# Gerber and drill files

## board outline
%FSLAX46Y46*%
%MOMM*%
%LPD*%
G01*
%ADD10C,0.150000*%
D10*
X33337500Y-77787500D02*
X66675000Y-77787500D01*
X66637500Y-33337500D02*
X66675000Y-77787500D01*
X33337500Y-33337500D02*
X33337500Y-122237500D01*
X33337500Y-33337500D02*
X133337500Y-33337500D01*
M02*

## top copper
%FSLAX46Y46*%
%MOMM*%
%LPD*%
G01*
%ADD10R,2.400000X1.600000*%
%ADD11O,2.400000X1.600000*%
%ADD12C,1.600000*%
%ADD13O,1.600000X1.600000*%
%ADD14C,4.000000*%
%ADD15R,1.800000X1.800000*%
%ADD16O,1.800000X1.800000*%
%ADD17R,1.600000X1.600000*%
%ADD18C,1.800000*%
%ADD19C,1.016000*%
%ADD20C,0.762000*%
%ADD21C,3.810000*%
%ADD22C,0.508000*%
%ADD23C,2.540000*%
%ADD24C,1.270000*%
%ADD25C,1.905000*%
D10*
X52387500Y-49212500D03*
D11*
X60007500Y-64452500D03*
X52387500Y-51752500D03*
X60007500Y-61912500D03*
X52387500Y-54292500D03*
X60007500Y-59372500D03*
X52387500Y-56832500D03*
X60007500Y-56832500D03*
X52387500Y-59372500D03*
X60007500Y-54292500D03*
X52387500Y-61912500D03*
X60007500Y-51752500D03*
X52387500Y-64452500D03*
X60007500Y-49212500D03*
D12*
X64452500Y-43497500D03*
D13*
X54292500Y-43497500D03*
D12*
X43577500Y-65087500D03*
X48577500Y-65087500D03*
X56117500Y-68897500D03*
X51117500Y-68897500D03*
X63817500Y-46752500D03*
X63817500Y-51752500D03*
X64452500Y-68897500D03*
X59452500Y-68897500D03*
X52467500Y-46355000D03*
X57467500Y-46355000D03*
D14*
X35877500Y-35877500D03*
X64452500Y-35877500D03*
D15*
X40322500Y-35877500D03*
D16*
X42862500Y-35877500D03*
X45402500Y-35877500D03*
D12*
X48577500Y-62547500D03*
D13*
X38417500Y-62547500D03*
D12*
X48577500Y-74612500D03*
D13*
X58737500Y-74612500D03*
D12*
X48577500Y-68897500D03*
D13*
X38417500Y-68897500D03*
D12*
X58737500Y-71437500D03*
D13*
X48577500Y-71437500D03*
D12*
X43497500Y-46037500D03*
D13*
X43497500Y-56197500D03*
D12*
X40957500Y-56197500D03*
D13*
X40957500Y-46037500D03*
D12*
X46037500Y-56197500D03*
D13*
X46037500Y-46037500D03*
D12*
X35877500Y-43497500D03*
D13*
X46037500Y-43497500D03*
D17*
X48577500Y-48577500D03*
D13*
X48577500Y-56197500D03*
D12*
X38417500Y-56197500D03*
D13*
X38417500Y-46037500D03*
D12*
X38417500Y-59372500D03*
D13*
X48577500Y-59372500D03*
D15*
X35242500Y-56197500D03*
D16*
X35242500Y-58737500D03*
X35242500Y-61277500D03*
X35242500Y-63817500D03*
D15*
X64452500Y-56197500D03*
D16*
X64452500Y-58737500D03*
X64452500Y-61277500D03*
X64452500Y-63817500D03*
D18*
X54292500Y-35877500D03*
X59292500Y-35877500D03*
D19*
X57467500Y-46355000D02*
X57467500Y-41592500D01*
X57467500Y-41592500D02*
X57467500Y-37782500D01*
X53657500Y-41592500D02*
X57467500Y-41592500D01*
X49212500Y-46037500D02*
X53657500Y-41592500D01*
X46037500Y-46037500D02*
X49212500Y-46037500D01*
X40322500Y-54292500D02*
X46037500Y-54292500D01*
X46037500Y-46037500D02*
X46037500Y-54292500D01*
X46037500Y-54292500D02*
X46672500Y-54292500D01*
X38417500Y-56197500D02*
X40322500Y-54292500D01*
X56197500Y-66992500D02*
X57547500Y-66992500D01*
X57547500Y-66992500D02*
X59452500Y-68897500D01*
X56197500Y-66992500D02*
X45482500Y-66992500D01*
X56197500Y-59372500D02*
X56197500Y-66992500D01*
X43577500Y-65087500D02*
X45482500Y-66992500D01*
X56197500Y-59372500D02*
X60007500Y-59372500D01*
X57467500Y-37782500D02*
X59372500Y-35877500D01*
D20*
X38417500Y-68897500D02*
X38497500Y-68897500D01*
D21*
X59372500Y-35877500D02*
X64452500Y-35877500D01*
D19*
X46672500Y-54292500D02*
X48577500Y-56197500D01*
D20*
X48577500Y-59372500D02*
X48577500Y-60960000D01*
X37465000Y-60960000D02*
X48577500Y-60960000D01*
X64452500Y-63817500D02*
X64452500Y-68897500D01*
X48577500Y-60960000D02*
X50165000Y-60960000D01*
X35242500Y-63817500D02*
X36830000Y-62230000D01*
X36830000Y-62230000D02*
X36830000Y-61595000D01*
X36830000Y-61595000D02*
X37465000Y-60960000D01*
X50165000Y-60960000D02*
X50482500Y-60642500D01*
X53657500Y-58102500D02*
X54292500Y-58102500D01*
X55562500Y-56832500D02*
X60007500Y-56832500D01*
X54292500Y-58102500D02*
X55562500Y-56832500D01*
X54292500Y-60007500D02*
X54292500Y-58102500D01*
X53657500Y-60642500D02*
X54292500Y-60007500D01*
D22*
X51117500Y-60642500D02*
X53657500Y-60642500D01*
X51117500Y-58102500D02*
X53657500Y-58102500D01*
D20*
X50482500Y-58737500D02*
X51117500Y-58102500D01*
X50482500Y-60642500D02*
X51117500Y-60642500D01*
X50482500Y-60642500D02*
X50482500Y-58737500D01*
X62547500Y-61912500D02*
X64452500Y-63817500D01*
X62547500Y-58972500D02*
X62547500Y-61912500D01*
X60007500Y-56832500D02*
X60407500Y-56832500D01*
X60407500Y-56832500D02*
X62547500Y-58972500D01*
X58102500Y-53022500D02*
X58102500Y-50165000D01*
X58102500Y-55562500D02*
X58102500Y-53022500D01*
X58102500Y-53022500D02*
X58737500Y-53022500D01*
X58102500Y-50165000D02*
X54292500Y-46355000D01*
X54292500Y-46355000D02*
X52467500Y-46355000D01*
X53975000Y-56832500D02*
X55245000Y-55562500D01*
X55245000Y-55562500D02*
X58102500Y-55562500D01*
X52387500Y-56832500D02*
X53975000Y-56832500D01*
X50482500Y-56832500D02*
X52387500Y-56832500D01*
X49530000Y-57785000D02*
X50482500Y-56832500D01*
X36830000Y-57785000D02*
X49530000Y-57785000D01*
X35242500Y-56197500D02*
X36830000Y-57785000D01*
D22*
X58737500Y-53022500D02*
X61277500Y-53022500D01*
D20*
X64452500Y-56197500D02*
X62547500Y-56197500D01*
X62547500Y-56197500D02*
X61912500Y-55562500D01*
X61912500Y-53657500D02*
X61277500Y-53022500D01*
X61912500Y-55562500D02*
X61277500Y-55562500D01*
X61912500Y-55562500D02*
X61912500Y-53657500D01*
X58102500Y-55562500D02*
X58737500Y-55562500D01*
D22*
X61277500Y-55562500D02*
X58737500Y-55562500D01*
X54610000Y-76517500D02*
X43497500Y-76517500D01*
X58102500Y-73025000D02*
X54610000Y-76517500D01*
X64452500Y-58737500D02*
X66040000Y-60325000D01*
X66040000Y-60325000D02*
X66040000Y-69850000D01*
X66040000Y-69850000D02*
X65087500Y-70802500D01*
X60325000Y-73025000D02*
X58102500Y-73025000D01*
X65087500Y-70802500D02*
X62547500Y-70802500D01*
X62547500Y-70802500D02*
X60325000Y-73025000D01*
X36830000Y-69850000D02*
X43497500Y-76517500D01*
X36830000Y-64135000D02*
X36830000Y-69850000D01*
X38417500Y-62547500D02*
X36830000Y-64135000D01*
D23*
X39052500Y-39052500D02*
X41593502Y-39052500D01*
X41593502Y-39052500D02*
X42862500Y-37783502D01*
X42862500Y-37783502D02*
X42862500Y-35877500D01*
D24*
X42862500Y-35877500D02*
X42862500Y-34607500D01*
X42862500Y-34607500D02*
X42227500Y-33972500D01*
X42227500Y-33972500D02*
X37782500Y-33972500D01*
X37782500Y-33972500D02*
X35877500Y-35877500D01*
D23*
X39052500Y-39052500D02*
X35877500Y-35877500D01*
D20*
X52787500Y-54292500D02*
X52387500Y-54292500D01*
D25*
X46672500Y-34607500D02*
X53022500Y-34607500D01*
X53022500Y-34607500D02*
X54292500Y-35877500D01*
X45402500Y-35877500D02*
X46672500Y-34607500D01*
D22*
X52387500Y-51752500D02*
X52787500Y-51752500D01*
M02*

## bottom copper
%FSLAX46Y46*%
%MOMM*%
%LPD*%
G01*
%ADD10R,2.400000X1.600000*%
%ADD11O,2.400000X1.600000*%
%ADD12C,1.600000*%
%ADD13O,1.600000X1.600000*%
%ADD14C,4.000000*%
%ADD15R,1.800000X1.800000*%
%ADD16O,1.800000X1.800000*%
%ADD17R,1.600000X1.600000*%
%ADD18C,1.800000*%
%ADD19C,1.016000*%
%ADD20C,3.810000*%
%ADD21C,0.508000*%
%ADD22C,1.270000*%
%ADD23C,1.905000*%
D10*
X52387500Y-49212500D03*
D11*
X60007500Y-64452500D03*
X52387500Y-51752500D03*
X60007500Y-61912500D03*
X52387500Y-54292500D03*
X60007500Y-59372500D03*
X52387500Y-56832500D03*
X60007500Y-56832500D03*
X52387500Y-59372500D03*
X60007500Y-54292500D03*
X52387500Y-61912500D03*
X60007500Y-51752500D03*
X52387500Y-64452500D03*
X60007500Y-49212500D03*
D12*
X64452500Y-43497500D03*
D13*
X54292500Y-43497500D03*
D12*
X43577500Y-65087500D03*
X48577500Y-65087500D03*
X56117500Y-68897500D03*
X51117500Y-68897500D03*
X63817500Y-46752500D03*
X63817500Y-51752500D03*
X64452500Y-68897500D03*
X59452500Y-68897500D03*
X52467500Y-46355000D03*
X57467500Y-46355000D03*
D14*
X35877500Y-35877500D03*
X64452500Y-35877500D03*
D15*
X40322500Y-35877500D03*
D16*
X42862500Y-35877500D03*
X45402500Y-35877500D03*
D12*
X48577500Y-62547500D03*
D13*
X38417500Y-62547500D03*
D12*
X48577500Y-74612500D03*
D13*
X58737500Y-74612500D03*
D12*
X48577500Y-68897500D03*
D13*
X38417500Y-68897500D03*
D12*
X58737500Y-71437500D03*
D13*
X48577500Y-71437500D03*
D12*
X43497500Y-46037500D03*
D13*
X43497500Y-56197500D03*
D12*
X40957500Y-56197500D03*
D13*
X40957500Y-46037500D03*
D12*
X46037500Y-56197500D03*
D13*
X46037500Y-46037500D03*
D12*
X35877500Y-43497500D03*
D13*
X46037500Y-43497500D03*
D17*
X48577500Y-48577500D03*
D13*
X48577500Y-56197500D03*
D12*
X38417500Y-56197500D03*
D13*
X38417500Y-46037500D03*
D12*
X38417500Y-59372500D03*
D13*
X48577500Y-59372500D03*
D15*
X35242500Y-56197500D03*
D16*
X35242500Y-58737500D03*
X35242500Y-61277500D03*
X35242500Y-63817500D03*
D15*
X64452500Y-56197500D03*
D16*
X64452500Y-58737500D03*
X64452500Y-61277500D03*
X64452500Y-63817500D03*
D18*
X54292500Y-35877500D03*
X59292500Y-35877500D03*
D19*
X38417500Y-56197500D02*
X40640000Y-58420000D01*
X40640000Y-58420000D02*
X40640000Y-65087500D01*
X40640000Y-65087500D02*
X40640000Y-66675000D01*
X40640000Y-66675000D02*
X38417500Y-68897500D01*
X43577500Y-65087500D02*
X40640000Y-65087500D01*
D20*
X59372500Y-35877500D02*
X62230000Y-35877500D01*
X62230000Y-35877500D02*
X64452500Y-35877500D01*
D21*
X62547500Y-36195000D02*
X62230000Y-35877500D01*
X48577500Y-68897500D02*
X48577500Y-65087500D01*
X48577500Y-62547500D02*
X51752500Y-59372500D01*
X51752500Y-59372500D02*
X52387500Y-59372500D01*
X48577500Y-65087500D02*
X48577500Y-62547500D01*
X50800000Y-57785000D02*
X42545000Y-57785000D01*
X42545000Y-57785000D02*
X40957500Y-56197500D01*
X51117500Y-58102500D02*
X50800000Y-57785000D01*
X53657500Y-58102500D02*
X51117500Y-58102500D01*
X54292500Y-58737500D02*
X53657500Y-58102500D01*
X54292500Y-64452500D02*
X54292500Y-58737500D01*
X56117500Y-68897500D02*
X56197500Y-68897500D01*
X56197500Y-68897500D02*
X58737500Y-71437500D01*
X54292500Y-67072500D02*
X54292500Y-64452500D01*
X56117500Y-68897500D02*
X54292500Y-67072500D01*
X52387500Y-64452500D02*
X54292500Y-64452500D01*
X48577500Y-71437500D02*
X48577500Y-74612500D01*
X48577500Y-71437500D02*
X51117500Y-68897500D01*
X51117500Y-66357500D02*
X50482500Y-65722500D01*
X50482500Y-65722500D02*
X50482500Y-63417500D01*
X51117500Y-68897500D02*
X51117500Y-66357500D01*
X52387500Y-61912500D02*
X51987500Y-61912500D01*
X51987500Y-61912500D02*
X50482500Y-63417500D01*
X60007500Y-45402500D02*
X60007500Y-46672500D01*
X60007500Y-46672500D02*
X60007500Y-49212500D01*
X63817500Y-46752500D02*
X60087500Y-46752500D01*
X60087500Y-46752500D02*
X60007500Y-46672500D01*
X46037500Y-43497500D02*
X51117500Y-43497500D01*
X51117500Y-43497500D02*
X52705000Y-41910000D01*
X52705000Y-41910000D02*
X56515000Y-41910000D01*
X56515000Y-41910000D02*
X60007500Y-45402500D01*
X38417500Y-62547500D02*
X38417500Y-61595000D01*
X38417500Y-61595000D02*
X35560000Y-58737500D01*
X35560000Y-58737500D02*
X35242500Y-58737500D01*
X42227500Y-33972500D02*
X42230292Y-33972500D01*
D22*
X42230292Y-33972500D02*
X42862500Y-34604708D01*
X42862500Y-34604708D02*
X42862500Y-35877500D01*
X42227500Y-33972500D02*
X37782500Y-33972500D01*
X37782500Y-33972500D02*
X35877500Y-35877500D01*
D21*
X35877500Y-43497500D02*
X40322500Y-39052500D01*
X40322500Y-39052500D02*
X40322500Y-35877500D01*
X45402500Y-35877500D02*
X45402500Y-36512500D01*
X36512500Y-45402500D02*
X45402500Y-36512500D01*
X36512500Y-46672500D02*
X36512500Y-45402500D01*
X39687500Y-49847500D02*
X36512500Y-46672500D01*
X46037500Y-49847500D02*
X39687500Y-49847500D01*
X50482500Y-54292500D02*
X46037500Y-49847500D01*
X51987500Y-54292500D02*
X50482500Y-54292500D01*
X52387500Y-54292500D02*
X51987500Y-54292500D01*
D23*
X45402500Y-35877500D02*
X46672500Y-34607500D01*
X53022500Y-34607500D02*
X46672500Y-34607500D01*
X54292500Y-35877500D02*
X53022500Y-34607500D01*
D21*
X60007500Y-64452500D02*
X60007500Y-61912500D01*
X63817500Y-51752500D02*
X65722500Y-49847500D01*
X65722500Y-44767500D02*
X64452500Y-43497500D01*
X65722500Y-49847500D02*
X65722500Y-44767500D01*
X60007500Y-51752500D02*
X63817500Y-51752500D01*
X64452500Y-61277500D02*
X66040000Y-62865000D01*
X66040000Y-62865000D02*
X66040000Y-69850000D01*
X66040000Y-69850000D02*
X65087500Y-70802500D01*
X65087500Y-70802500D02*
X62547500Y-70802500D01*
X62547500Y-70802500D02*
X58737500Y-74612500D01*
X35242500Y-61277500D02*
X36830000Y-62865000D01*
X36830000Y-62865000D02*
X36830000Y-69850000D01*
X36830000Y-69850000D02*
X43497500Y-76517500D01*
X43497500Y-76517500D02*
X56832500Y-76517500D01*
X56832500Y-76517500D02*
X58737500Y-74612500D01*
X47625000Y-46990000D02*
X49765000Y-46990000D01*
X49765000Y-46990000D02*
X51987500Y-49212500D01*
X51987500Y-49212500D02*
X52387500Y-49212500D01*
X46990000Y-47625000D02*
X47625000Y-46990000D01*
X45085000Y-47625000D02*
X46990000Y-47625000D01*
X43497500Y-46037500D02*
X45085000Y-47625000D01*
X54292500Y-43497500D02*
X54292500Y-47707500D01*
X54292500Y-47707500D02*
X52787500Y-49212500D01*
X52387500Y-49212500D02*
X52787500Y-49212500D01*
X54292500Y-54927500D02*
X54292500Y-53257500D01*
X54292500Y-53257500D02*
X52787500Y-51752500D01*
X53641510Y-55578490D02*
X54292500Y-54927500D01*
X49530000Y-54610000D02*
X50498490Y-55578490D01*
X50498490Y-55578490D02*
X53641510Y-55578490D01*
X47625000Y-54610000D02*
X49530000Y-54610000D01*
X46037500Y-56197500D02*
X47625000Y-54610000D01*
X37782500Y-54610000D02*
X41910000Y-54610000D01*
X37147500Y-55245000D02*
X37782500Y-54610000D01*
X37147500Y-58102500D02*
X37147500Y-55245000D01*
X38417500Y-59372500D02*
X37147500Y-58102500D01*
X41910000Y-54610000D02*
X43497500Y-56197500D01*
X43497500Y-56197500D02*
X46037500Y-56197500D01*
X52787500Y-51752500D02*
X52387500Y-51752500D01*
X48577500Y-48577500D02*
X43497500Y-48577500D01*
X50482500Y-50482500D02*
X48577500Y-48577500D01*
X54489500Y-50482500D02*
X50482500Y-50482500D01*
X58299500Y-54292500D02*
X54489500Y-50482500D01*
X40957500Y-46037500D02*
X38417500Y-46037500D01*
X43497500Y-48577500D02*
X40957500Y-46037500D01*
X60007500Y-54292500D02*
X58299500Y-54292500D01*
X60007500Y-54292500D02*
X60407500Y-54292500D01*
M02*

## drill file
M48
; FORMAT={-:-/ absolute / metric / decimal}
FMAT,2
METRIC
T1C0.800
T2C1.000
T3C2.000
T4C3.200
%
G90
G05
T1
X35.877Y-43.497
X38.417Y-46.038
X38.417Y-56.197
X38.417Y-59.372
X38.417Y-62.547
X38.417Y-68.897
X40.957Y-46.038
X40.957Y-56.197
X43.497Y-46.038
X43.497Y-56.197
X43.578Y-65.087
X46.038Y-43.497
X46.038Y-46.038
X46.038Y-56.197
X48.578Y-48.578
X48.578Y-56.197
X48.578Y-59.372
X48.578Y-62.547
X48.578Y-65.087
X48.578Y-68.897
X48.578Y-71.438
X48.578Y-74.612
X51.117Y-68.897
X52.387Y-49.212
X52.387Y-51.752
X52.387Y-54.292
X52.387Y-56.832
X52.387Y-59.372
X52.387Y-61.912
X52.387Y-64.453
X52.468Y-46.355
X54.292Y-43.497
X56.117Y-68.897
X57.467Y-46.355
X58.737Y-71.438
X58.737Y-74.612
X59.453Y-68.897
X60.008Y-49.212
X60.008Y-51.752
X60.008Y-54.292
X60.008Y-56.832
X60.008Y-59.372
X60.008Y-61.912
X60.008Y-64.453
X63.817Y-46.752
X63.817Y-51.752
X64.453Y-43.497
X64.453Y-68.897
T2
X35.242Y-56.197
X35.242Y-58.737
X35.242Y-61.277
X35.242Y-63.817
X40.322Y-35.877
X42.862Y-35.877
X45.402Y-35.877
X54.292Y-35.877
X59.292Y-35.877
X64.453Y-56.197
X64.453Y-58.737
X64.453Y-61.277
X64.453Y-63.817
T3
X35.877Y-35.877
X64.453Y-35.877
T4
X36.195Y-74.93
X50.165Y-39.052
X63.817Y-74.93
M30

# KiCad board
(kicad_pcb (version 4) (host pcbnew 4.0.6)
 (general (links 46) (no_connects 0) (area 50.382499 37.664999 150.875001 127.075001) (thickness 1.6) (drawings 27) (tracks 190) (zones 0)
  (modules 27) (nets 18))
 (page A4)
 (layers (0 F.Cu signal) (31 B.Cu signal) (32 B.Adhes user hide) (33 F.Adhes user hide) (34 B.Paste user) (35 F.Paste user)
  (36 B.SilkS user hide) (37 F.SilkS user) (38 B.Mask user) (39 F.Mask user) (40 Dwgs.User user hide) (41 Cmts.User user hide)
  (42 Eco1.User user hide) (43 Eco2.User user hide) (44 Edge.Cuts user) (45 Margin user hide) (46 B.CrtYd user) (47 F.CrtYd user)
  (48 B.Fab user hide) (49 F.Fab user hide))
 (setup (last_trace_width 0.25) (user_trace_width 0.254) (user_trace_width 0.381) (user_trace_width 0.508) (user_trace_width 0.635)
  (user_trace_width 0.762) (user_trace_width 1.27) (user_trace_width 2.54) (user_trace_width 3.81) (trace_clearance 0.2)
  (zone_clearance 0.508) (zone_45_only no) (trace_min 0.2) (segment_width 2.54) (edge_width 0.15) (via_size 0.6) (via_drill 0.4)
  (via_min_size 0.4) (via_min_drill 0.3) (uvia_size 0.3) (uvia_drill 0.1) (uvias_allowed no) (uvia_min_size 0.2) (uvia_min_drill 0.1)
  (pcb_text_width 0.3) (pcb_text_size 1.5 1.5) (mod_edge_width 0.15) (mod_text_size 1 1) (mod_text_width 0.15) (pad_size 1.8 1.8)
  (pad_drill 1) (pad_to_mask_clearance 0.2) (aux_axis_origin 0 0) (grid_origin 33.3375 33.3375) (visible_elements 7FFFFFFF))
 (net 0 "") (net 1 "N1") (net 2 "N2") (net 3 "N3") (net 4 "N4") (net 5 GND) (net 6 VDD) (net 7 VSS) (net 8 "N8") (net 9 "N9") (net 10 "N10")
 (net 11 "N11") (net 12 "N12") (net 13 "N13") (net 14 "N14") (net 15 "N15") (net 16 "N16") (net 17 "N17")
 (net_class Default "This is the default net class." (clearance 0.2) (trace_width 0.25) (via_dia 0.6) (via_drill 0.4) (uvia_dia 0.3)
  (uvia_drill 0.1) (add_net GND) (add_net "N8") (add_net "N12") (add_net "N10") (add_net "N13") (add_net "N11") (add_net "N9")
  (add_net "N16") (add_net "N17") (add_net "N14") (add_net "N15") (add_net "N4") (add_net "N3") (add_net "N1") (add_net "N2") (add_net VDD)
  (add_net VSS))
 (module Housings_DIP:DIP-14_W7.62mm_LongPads (layer F.Cu) (at 52.3875 49.2125)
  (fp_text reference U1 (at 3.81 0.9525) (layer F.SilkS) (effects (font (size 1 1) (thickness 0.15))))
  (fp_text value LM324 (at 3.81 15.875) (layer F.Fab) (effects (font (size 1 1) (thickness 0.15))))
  (pad 1 thru_hole rect (at 0 0) (size 2.4 1.6) (drill 0.8) (layers *.Cu *.Mask) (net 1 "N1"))
  (pad 8 thru_hole oval (at 7.62 15.24) (size 2.4 1.6) (drill 0.8) (layers *.Cu *.Mask) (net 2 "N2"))
  (pad 2 thru_hole oval (at 0 2.54) (size 2.4 1.6) (drill 0.8) (layers *.Cu *.Mask) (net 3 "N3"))
  (pad 9 thru_hole oval (at 7.62 12.7) (size 2.4 1.6) (drill 0.8) (layers *.Cu *.Mask) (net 2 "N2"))
  (pad 3 thru_hole oval (at 0 5.08) (size 2.4 1.6) (drill 0.8) (layers *.Cu *.Mask) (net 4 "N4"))
  (pad 10 thru_hole oval (at 7.62 10.16) (size 2.4 1.6) (drill 0.8) (layers *.Cu *.Mask) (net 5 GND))
  (pad 4 thru_hole oval (at 0 7.62) (size 2.4 1.6) (drill 0.8) (layers *.Cu *.Mask) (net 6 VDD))
  (pad 11 thru_hole oval (at 7.62 7.62) (size 2.4 1.6) (drill 0.8) (layers *.Cu *.Mask) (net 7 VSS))
  (pad 5 thru_hole oval (at 0 10.16) (size 2.4 1.6) (drill 0.8) (layers *.Cu *.Mask) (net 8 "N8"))
  (pad 12 thru_hole oval (at 7.62 5.08) (size 2.4 1.6) (drill 0.8) (layers *.Cu *.Mask) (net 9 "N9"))
  (pad 6 thru_hole oval (at 0 12.7) (size 2.4 1.6) (drill 0.8) (layers *.Cu *.Mask) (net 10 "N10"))
  (pad 13 thru_hole oval (at 7.62 2.54) (size 2.4 1.6) (drill 0.8) (layers *.Cu *.Mask) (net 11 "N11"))
  (pad 7 thru_hole oval (at 0 15.24) (size 2.4 1.6) (drill 0.8) (layers *.Cu *.Mask) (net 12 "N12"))
  (pad 14 thru_hole oval (at 7.62 0) (size 2.4 1.6) (drill 0.8) (layers *.Cu *.Mask) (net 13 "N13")))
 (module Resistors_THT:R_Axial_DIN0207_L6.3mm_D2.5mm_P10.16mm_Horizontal (layer F.Cu) (at 64.4525 43.4975 180)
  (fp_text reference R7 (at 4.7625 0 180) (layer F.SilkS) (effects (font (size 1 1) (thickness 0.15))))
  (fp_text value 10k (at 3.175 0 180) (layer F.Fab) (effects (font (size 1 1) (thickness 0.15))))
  (pad 1 thru_hole circle (at 0 0 180) (size 1.6 1.6) (drill 0.8) (layers *.Cu *.Mask) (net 11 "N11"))
  (pad 2 thru_hole oval (at 10.16 0 180) (size 1.6 1.6) (drill 0.8) (layers *.Cu *.Mask) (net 1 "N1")))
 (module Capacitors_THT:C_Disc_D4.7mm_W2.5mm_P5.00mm (layer F.Cu) (at 43.5775 65.0875)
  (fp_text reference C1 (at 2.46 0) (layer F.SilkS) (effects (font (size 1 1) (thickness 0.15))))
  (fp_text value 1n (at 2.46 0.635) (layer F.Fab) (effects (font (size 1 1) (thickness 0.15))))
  (pad 1 thru_hole circle (at 0 0) (size 1.6 1.6) (drill 0.8) (layers *.Cu *.Mask) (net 5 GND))
  (pad 2 thru_hole circle (at 5 0) (size 1.6 1.6) (drill 0.8) (layers *.Cu *.Mask) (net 8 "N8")))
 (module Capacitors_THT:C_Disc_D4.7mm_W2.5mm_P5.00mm (layer F.Cu) (at 56.1175 68.8975 180)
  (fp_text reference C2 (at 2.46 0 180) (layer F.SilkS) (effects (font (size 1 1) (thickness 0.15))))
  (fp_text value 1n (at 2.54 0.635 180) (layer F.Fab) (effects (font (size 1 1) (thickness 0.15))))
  (pad 1 thru_hole circle (at 0 0 180) (size 1.6 1.6) (drill 0.8) (layers *.Cu *.Mask) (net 12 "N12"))
  (pad 2 thru_hole circle (at 5 0 180) (size 1.6 1.6) (drill 0.8) (layers *.Cu *.Mask) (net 10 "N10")))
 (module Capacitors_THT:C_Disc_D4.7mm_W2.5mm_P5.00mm (layer F.Cu) (at 63.8175 46.7525 270)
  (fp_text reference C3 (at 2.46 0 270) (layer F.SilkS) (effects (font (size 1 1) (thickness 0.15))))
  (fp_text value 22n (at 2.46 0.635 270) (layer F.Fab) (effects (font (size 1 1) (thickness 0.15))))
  (pad 1 thru_hole circle (at 0 0 270) (size 1.6 1.6) (drill 0.8) (layers *.Cu *.Mask) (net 13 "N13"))
  (pad 2 thru_hole circle (at 5 0 270) (size 1.6 1.6) (drill 0.8) (layers *.Cu *.Mask) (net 11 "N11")))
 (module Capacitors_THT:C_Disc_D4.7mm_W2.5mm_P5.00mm (layer F.Cu) (at 64.4525 68.8975 180)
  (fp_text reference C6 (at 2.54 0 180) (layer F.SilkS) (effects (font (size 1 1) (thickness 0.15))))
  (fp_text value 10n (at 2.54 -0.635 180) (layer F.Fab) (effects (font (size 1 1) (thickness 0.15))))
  (pad 1 thru_hole circle (at 0 0 180) (size 1.6 1.6) (drill 0.8) (layers *.Cu *.Mask) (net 7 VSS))
  (pad 2 thru_hole circle (at 5 0 180) (size 1.6 1.6) (drill 0.8) (layers *.Cu *.Mask) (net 5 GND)))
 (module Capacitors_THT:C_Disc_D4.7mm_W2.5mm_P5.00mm (layer F.Cu) (at 52.4675 46.355)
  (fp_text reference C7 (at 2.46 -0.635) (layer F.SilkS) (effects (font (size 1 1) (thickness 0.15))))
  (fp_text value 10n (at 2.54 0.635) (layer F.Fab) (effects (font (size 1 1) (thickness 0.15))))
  (pad 1 thru_hole circle (at 0 0) (size 1.6 1.6) (drill 0.8) (layers *.Cu *.Mask) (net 6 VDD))
  (pad 2 thru_hole circle (at 5 0) (size 1.6 1.6) (drill 0.8) (layers *.Cu *.Mask) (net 5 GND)))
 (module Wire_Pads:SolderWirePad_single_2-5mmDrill (layer F.Cu) (at 35.8775 35.8775)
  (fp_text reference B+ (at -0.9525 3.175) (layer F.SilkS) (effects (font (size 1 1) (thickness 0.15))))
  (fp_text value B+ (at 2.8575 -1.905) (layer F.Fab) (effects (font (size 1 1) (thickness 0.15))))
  (pad 1 thru_hole circle (at 0 0) (size 4 4) (drill 2) (layers *.Cu *.Mask) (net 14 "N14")))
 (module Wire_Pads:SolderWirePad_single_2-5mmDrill (layer F.Cu) (at 64.4525 35.8775)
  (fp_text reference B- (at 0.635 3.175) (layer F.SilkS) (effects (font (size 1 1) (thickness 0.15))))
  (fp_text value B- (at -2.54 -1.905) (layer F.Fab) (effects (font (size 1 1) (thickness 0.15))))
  (pad 1 thru_hole circle (at 0 0) (size 4 4) (drill 2) (layers *.Cu *.Mask) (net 5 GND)))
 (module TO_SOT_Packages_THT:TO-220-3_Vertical (layer F.Cu) (at 40.3225 35.8775)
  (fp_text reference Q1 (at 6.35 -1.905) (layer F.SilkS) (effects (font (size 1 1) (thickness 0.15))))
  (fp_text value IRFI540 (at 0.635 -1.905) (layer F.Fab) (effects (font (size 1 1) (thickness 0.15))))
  (pad 1 thru_hole rect (at 0 0) (size 1.8 1.8) (drill 1) (layers *.Cu *.Mask) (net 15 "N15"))
  (pad 2 thru_hole oval (at 2.54 0) (size 1.8 1.8) (drill 1) (layers *.Cu *.Mask) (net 14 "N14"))
  (pad 3 thru_hole oval (at 5.08 0) (size 1.8 1.8) (drill 1) (layers *.Cu *.Mask) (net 4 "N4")))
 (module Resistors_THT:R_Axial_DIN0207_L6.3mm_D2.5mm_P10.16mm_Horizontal (layer F.Cu) (at 48.5775 62.5475 180)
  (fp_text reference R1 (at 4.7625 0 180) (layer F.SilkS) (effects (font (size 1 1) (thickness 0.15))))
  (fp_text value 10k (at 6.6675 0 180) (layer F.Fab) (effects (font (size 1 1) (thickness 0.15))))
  (pad 1 thru_hole circle (at 0 0 180) (size 1.6 1.6) (drill 0.8) (layers *.Cu *.Mask) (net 8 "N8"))
  (pad 2 thru_hole oval (at 10.16 0 180) (size 1.6 1.6) (drill 0.8) (layers *.Cu *.Mask) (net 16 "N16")))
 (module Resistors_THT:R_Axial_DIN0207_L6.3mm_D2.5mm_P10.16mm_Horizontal (layer F.Cu) (at 48.5775 74.6125)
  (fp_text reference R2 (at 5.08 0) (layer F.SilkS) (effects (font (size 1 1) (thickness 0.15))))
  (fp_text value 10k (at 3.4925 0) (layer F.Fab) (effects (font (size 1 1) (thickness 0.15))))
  (pad 1 thru_hole circle (at 0 0) (size 1.6 1.6) (drill 0.8) (layers *.Cu *.Mask) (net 10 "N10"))
  (pad 2 thru_hole oval (at 10.16 0) (size 1.6 1.6) (drill 0.8) (layers *.Cu *.Mask) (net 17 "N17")))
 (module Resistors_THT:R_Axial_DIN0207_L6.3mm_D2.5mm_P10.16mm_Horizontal (layer F.Cu) (at 48.5775 68.8975 180)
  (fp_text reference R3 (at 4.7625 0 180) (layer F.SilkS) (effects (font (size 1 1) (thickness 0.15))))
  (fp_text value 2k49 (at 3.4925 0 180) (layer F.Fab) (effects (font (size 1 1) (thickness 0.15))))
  (pad 1 thru_hole circle (at 0 0 180) (size 1.6 1.6) (drill 0.8) (layers *.Cu *.Mask) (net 8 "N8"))
  (pad 2 thru_hole oval (at 10.16 0 180) (size 1.6 1.6) (drill 0.8) (layers *.Cu *.Mask) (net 5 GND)))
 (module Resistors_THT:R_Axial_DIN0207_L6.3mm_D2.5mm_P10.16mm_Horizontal (layer F.Cu) (at 58.7375 71.4375 180)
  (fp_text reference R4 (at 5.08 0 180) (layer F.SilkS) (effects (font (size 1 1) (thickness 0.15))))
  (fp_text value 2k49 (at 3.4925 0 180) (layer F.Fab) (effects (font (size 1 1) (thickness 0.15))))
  (pad 1 thru_hole circle (at 0 0 180) (size 1.6 1.6) (drill 0.8) (layers *.Cu *.Mask) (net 12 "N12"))
  (pad 2 thru_hole oval (at 10.16 0 180) (size 1.6 1.6) (drill 0.8) (layers *.Cu *.Mask) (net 10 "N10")))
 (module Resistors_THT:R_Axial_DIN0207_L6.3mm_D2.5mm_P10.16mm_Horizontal (layer F.Cu) (at 43.4975 46.0375 270)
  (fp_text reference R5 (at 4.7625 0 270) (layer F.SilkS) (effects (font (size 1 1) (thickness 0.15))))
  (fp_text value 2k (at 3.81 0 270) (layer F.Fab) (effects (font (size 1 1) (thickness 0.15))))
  (pad 1 thru_hole circle (at 0 0 270) (size 1.6 1.6) (drill 0.8) (layers *.Cu *.Mask) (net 1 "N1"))
  (pad 2 thru_hole oval (at 10.16 0 270) (size 1.6 1.6) (drill 0.8) (layers *.Cu *.Mask) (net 3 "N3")))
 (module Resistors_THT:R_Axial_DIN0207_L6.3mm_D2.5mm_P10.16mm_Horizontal (layer F.Cu) (at 40.9575 56.1975 90)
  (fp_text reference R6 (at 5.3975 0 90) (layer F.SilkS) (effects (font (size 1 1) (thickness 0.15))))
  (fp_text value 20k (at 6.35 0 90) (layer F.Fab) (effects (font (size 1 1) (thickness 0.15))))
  (pad 1 thru_hole circle (at 0 0 90) (size 1.6 1.6) (drill 0.8) (layers *.Cu *.Mask) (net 12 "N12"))
  (pad 2 thru_hole oval (at 10.16 0 90) (size 1.6 1.6) (drill 0.8) (layers *.Cu *.Mask) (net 9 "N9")))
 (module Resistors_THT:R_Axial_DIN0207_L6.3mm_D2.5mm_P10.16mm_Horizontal (layer F.Cu) (at 46.0375 56.1975 90)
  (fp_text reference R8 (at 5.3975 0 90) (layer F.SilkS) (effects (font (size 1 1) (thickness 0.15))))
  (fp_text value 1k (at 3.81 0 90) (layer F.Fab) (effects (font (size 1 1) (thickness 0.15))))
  (pad 1 thru_hole circle (at 0 0 90) (size 1.6 1.6) (drill 0.8) (layers *.Cu *.Mask) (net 3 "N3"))
  (pad 2 thru_hole oval (at 10.16 0 90) (size 1.6 1.6) (drill 0.8) (layers *.Cu *.Mask) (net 5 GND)))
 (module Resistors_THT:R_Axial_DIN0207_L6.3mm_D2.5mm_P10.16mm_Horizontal (layer F.Cu) (at 35.8775 43.4975)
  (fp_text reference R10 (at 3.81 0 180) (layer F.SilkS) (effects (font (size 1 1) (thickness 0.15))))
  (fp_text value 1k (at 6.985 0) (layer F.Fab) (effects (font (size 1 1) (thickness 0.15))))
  (pad 1 thru_hole circle (at 0 0) (size 1.6 1.6) (drill 0.8) (layers *.Cu *.Mask) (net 15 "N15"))
  (pad 2 thru_hole oval (at 10.16 0) (size 1.6 1.6) (drill 0.8) (layers *.Cu *.Mask) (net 13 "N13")))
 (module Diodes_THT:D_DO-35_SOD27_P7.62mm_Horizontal (layer F.Cu) (at 48.5775 48.5775 270)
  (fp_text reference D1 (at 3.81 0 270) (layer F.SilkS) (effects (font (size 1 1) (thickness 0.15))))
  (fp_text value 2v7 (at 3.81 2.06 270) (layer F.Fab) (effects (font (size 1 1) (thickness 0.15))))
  (pad 1 thru_hole rect (at 0 0 270) (size 1.6 1.6) (drill 0.8) (layers *.Cu *.Mask) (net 9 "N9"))
  (pad 2 thru_hole oval (at 7.62 0 270) (size 1.6 1.6) (drill 0.8) (layers *.Cu *.Mask) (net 5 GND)))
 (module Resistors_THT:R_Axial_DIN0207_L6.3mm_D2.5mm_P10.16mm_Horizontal (layer F.Cu) (at 38.4175 56.1975 90)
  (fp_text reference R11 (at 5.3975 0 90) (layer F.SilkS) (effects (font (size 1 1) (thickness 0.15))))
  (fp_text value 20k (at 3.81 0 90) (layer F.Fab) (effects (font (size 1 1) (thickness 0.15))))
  (pad 1 thru_hole circle (at 0 0 90) (size 1.6 1.6) (drill 0.8) (layers *.Cu *.Mask) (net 5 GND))
  (pad 2 thru_hole oval (at 10.16 0 90) (size 1.6 1.6) (drill 0.8) (layers *.Cu *.Mask) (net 9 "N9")))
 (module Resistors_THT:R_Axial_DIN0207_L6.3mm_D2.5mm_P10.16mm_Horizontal (layer F.Cu) (at 38.4175 59.3725)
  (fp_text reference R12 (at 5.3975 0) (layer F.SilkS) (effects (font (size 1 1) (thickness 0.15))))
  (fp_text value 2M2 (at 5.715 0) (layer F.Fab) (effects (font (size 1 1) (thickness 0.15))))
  (pad 1 thru_hole circle (at 0 0) (size 1.6 1.6) (drill 0.8) (layers *.Cu *.Mask) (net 3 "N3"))
  (pad 2 thru_hole oval (at 10.16 0) (size 1.6 1.6) (drill 0.8) (layers *.Cu *.Mask) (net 7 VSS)))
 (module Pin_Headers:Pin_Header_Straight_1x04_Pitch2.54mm (layer F.Cu) (at 35.2425 56.1975)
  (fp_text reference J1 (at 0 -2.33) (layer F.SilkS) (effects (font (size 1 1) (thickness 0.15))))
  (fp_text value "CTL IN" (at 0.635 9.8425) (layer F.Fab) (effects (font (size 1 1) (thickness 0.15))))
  (pad 1 thru_hole rect (at 0 0) (size 1.8 1.8) (drill 1) (layers *.Cu *.Mask) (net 6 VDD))
  (pad 2 thru_hole oval (at 0 2.54) (size 1.8 1.8) (drill 1) (layers *.Cu *.Mask) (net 16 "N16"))
  (pad 3 thru_hole oval (at 0 5.08) (size 1.8 1.8) (drill 1) (layers *.Cu *.Mask) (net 17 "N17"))
  (pad 4 thru_hole oval (at 0 7.62) (size 1.8 1.8) (drill 1) (layers *.Cu *.Mask) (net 7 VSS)))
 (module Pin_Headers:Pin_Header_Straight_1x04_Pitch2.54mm (layer F.Cu) (at 64.4525 56.1975)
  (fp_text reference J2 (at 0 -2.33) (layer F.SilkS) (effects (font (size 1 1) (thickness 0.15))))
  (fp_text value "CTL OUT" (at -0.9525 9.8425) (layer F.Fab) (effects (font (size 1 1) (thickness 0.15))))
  (pad 1 thru_hole rect (at 0 0) (size 1.8 1.8) (drill 1) (layers *.Cu *.Mask) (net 6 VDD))
  (pad 2 thru_hole oval (at 0 2.54) (size 1.8 1.8) (drill 1) (layers *.Cu *.Mask) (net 16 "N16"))
  (pad 3 thru_hole oval (at 0 5.08) (size 1.8 1.8) (drill 1) (layers *.Cu *.Mask) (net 17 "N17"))
  (pad 4 thru_hole oval (at 0 7.62) (size 1.8 1.8) (drill 1) (layers *.Cu *.Mask) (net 7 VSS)))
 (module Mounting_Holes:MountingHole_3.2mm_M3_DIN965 (layer F.Cu) (at 50.165 39.0525)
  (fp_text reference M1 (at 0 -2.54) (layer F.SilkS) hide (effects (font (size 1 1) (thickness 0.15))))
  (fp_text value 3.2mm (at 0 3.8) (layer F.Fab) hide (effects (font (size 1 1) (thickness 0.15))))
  (pad "" np_thru_hole circle (at 0 0) (size 3.2 3.2) (drill 3.2) (layers *.Cu *.Mask)))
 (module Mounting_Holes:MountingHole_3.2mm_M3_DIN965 (layer F.Cu) (at 36.195 74.93)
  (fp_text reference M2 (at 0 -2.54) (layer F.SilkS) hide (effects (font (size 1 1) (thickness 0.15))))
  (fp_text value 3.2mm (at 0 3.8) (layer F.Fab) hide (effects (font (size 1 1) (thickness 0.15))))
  (pad 1 np_thru_hole circle (at 0 0) (size 3.2 3.2) (drill 3.2) (layers *.Cu *.Mask)))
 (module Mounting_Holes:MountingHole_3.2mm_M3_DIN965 (layer F.Cu) (at 63.8175 74.93)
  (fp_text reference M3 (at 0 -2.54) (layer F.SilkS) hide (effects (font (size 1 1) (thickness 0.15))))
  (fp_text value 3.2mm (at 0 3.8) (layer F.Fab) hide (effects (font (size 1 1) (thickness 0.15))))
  (pad 1 np_thru_hole circle (at 0 0) (size 3.2 3.2) (drill 3.2) (layers *.Cu *.Mask)))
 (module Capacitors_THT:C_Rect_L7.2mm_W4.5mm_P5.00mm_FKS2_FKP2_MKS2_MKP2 (layer F.Cu) (at 54.2925 35.8775)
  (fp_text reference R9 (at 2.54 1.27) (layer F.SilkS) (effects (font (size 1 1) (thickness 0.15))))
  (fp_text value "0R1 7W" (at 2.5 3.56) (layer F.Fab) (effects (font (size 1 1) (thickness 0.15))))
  (pad 1 thru_hole circle (at 0 0) (size 1.8 1.8) (drill 1) (layers *.Cu *.Mask) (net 4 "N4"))
  (pad 2 thru_hole circle (at 5 0) (size 1.8 1.8) (drill 1) (layers *.Cu *.Mask) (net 5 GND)))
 (gr_line (start 33.3375 77.7875) (end 66.675 77.7875) (layer Edge.Cuts) (width 0.15))
 (gr_line (start 66.6375 33.3375) (end 66.675 77.7875) (layer Edge.Cuts) (width 0.15))
 (gr_line (start 33.3375 33.3375) (end 33.3375 122.2375) (layer Edge.Cuts) (width 0.15))
 (gr_line (start 33.3375 33.3375) (end 133.3375 33.3375) (layer Edge.Cuts) (width 0.15))
 (segment (start 57.4675 46.355) (end 57.4675 41.5925) (width 1.016) (layer F.Cu) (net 5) (status 10))
 (segment (start 57.4675 41.5925) (end 57.4675 37.7825) (width 1.016) (layer F.Cu) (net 5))
 (segment (start 53.6575 41.5925) (end 57.4675 41.5925) (width 1.016) (layer F.Cu) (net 5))
 (segment (start 49.2125 46.0375) (end 53.6575 41.5925) (width 1.016) (layer F.Cu) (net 5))
 (segment (start 46.0375 46.0375) (end 49.2125 46.0375) (width 1.016) (layer F.Cu) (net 5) (status 10))
 (segment (start 40.3225 54.2925) (end 46.0375 54.2925) (width 1.016) (layer F.Cu) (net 5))
 (segment (start 46.0375 46.0375) (end 46.0375 54.2925) (width 1.016) (layer F.Cu) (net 5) (status 10))
 (segment (start 46.0375 54.2925) (end 46.6725 54.2925) (width 1.016) (layer F.Cu) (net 5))
 (segment (start 38.4175 56.1975) (end 40.3225 54.2925) (width 1.016) (layer F.Cu) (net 5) (status 10))
 (segment (start 38.4175 56.1975) (end 40.64 58.42) (width 1.016) (layer B.Cu) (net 5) (status 10))
 (segment (start 40.64 58.42) (end 40.64 65.0875) (width 1.016) (layer B.Cu) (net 5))
 (segment (start 56.1975 66.9925) (end 57.5475 66.9925) (width 1.016) (layer F.Cu) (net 5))
 (segment (start 57.5475 66.9925) (end 59.4525 68.8975) (width 1.016) (layer F.Cu) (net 5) (status 20))
 (segment (start 56.1975 66.9925) (end 45.4825 66.9925) (width 1.016) (layer F.Cu) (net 5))
 (segment (start 56.1975 59.3725) (end 56.1975 66.9925) (width 1.016) (layer F.Cu) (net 5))
 (segment (start 43.5775 65.0875) (end 45.4825 66.9925) (width 1.016) (layer F.Cu) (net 5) (status 10))
 (segment (start 40.64 65.0875) (end 40.64 66.675) (width 1.016) (layer B.Cu) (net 5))
 (segment (start 40.64 66.675) (end 38.4175 68.8975) (width 1.016) (layer B.Cu) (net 5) (status 20))
 (segment (start 56.1975 59.3725) (end 60.0075 59.3725) (width 1.016) (layer F.Cu) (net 5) (status 20))
 (segment (start 43.5775 65.0875) (end 40.64 65.0875) (width 1.016) (layer B.Cu) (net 5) (status 10))
 (segment (start 57.4675 37.7825) (end 59.3725 35.8775) (width 1.016) (layer F.Cu) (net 5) (status 20))
 (segment (start 38.4175 68.8975) (end 38.4975 68.8975) (width 0.762) (layer F.Cu) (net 5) (status 30))
 (segment (start 59.3725 35.8775) (end 64.4525 35.8775) (width 3.81) (layer F.Cu) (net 5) (status 30))
 (segment (start 59.3725 35.8775) (end 62.23 35.8775) (width 3.81) (layer B.Cu) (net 5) (status 10))
 (segment (start 62.23 35.8775) (end 64.4525 35.8775) (width 3.81) (layer B.Cu) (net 5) (status 20))
 (segment (start 62.5475 36.195) (end 62.23 35.8775) (width 0.508) (layer B.Cu) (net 5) (status 10))
 (segment (start 46.6725 54.2925) (end 48.5775 56.1975) (width 1.016) (layer F.Cu) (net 5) (status 20))
 (segment (start 48.5775 68.8975) (end 48.5775 65.0875) (width 0.508) (layer B.Cu) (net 8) (status 30))
 (segment (start 48.5775 62.5475) (end 51.7525 59.3725) (width 0.508) (layer B.Cu) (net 8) (status 30))
 (segment (start 51.7525 59.3725) (end 52.3875 59.3725) (width 0.508) (layer B.Cu) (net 8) (status 30))
 (segment (start 48.5775 65.0875) (end 48.5775 62.5475) (width 0.508) (layer B.Cu) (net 8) (status 30))
 (segment (start 50.8 57.785) (end 42.545 57.785) (width 0.508) (layer B.Cu) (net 12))
 (segment (start 42.545 57.785) (end 40.9575 56.1975) (width 0.508) (layer B.Cu) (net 12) (status 20))
 (segment (start 51.1175 58.1025) (end 50.8 57.785) (width 0.508) (layer B.Cu) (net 12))
 (segment (start 53.6575 58.1025) (end 51.1175 58.1025) (width 0.508) (layer B.Cu) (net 12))
 (segment (start 54.2925 58.7375) (end 53.6575 58.1025) (width 0.508) (layer B.Cu) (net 12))
 (segment (start 54.2925 64.4525) (end 54.2925 58.7375) (width 0.508) (layer B.Cu) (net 12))
 (segment (start 56.1175 68.8975) (end 56.1975 68.8975) (width 0.508) (layer B.Cu) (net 12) (status 30))
 (segment (start 56.1975 68.8975) (end 58.7375 71.4375) (width 0.508) (layer B.Cu) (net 12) (status 30))
 (segment (start 54.2925 67.0725) (end 54.2925 64.4525) (width 0.508) (layer B.Cu) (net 12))
 (segment (start 56.1175 68.8975) (end 54.2925 67.0725) (width 0.508) (layer B.Cu) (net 12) (status 10))
 (segment (start 52.3875 64.4525) (end 54.2925 64.4525) (width 0.508) (layer B.Cu) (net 12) (status 10))
 (segment (start 48.5775 71.4375) (end 48.5775 74.6125) (width 0.508) (layer B.Cu) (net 10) (status 30))
 (segment (start 48.5775 71.4375) (end 51.1175 68.8975) (width 0.508) (layer B.Cu) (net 10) (status 30))
 (segment (start 51.1175 66.3575) (end 50.4825 65.7225) (width 0.508) (layer B.Cu) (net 10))
 (segment (start 50.4825 65.7225) (end 50.4825 63.4175) (width 0.508) (layer B.Cu) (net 10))
 (segment (start 51.1175 68.8975) (end 51.1175 66.3575) (width 0.508) (layer B.Cu) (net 10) (status 10))
 (segment (start 52.3875 61.9125) (end 51.9875 61.9125) (width 0.508) (layer B.Cu) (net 10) (status 30))
 (segment (start 51.9875 61.9125) (end 50.4825 63.4175) (width 0.508) (layer B.Cu) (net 10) (status 10))
 (segment (start 60.0075 45.4025) (end 60.0075 46.6725) (width 0.508) (layer B.Cu) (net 13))
 (segment (start 60.0075 46.6725) (end 60.0075 49.2125) (width 0.508) (layer B.Cu) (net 13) (status 20))
 (segment (start 63.8175 46.7525) (end 60.0875 46.7525) (width 0.508) (layer B.Cu) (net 13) (status 10))
 (segment (start 60.0875 46.7525) (end 60.0075 46.6725) (width 0.508) (layer B.Cu) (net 13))
 (segment (start 46.0375 43.4975) (end 51.1175 43.4975) (width 0.508) (layer B.Cu) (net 13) (status 10))
 (segment (start 51.1175 43.4975) (end 52.705 41.91) (width 0.508) (layer B.Cu) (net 13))
 (segment (start 52.705 41.91) (end 56.515 41.91) (width 0.508) (layer B.Cu) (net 13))
 (segment (start 56.515 41.91) (end 60.0075 45.4025) (width 0.508) (layer B.Cu) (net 13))
 (segment (start 48.5775 59.3725) (end 48.5775 60.96) (width 0.762) (layer F.Cu) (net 7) (status 10))
 (segment (start 37.465 60.96) (end 48.5775 60.96) (width 0.762) (layer F.Cu) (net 7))
 (segment (start 64.4525 63.8175) (end 64.4525 68.8975) (width 0.762) (layer F.Cu) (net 7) (status 30))
 (segment (start 48.5775 60.96) (end 50.165 60.96) (width 0.762) (layer F.Cu) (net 7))
 (segment (start 35.2425 63.8175) (end 36.83 62.23) (width 0.762) (layer F.Cu) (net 7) (status 10))
 (segment (start 36.83 62.23) (end 36.83 61.595) (width 0.762) (layer F.Cu) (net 7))
 (segment (start 36.83 61.595) (end 37.465 60.96) (width 0.762) (layer F.Cu) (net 7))
 (segment (start 50.165 60.96) (end 50.4825 60.6425) (width 0.762) (layer F.Cu) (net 7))
 (segment (start 53.6575 58.1025) (end 54.2925 58.1025) (width 0.762) (layer F.Cu) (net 7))
 (segment (start 55.5625 56.8325) (end 60.0075 56.8325) (width 0.762) (layer F.Cu) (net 7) (status 20))
 (segment (start 54.2925 58.1025) (end 55.5625 56.8325) (width 0.762) (layer F.Cu) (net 7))
 (segment (start 54.2925 60.0075) (end 54.2925 58.1025) (width 0.762) (layer F.Cu) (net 7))
 (segment (start 53.6575 60.6425) (end 54.2925 60.0075) (width 0.762) (layer F.Cu) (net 7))
 (segment (start 51.1175 60.6425) (end 53.6575 60.6425) (width 0.508) (layer F.Cu) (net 7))
 (segment (start 51.1175 58.1025) (end 53.6575 58.1025) (width 0.508) (layer F.Cu) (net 7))
 (segment (start 50.4825 58.7375) (end 51.1175 58.1025) (width 0.762) (layer F.Cu) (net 7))
 (segment (start 50.4825 60.6425) (end 51.1175 60.6425) (width 0.762) (layer F.Cu) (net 7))
 (segment (start 50.4825 60.6425) (end 50.4825 58.7375) (width 0.762) (layer F.Cu) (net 7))
 (segment (start 62.5475 61.9125) (end 64.4525 63.8175) (width 0.762) (layer F.Cu) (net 7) (status 20))
 (segment (start 62.5475 58.9725) (end 62.5475 61.9125) (width 0.762) (layer F.Cu) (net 7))
 (segment (start 60.0075 56.8325) (end 60.4075 56.8325) (width 0.762) (layer F.Cu) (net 7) (status 30))
 (segment (start 60.4075 56.8325) (end 62.5475 58.9725) (width 0.762) (layer F.Cu) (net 7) (status 10))
 (segment (start 58.1025 53.0225) (end 58.1025 50.165) (width 0.762) (layer F.Cu) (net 6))
 (segment (start 58.1025 55.5625) (end 58.1025 53.0225) (width 0.762) (layer F.Cu) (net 6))
 (segment (start 58.1025 53.0225) (end 58.7375 53.0225) (width 0.762) (layer F.Cu) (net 6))
 (segment (start 58.1025 50.165) (end 54.2925 46.355) (width 0.762) (layer F.Cu) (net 6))
 (segment (start 54.2925 46.355) (end 52.4675 46.355) (width 0.762) (layer F.Cu) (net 6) (status 20))
 (segment (start 53.975 56.8325) (end 55.245 55.5625) (width 0.762) (layer F.Cu) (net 6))
 (segment (start 55.245 55.5625) (end 58.1025 55.5625) (width 0.762) (layer F.Cu) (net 6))
 (segment (start 52.3875 56.8325) (end 53.975 56.8325) (width 0.762) (layer F.Cu) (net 6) (status 10))
 (segment (start 50.4825 56.8325) (end 52.3875 56.8325) (width 0.762) (layer F.Cu) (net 6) (status 20))
 (segment (start 49.53 57.785) (end 50.4825 56.8325) (width 0.762) (layer F.Cu) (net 6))
 (segment (start 36.83 57.785) (end 49.53 57.785) (width 0.762) (layer F.Cu) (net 6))
 (segment (start 35.2425 56.1975) (end 36.83 57.785) (width 0.762) (layer F.Cu) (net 6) (status 10))
 (segment (start 58.7375 53.0225) (end 61.2775 53.0225) (width 0.508) (layer F.Cu) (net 6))
 (segment (start 64.4525 56.1975) (end 62.5475 56.1975) (width 0.762) (layer F.Cu) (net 6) (status 10))
 (segment (start 62.5475 56.1975) (end 61.9125 55.5625) (width 0.762) (layer F.Cu) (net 6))
 (segment (start 61.9125 53.6575) (end 61.2775 53.0225) (width 0.762) (layer F.Cu) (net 6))
 (segment (start 61.9125 55.5625) (end 61.2775 55.5625) (width 0.762) (layer F.Cu) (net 6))
 (segment (start 61.9125 55.5625) (end 61.9125 53.6575) (width 0.762) (layer F.Cu) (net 6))
 (segment (start 58.1025 55.5625) (end 58.7375 55.5625) (width 0.762) (layer F.Cu) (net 6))
 (segment (start 61.2775 55.5625) (end 58.7375 55.5625) (width 0.508) (layer F.Cu) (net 6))
 (segment (start 54.61 76.5175) (end 43.4975 76.5175) (width 0.508) (layer F.Cu) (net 16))
 (segment (start 58.1025 73.025) (end 54.61 76.5175) (width 0.508) (layer F.Cu) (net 16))
 (segment (start 64.4525 58.7375) (end 66.04 60.325) (width 0.508) (layer F.Cu) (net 16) (status 10))
 (segment (start 66.04 60.325) (end 66.04 69.85) (width 0.508) (layer F.Cu) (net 16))
 (segment (start 66.04 69.85) (end 65.0875 70.8025) (width 0.508) (layer F.Cu) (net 16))
 (segment (start 60.325 73.025) (end 58.1025 73.025) (width 0.508) (layer F.Cu) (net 16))
 (segment (start 65.0875 70.8025) (end 62.5475 70.8025) (width 0.508) (layer F.Cu) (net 16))
 (segment (start 62.5475 70.8025) (end 60.325 73.025) (width 0.508) (layer F.Cu) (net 16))
 (segment (start 36.83 69.85) (end 43.4975 76.5175) (width 0.508) (layer F.Cu) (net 16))
 (segment (start 36.83 64.135) (end 36.83 69.85) (width 0.508) (layer F.Cu) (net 16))
 (segment (start 38.4175 62.5475) (end 36.83 64.135) (width 0.508) (layer F.Cu) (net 16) (status 10))
 (segment (start 38.4175 62.5475) (end 38.4175 61.595) (width 0.508) (layer B.Cu) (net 16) (status 10))
 (segment (start 38.4175 61.595) (end 35.56 58.7375) (width 0.508) (layer B.Cu) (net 16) (status 20))
 (segment (start 35.56 58.7375) (end 35.2425 58.7375) (width 0.508) (layer B.Cu) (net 16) (status 30))
 (segment (start 39.0525 39.0525) (end 41.593502 39.0525) (width 2.54) (layer F.Cu) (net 14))
 (segment (start 41.593502 39.0525) (end 42.8625 37.783502) (width 2.54) (layer F.Cu) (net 14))
 (segment (start 42.8625 37.783502) (end 42.8625 35.8775) (width 2.54) (layer F.Cu) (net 14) (status 20))
 (segment (start 42.8625 35.8775) (end 42.8625 34.6075) (width 1.27) (layer F.Cu) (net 14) (status 10))
 (segment (start 42.2275 33.9725) (end 42.230292 33.9725) (width 0.508) (layer B.Cu) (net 14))
 (segment (start 42.230292 33.9725) (end 42.8625 34.604708) (width 1.27) (layer B.Cu) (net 14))
 (segment (start 42.8625 34.604708) (end 42.8625 35.8775) (width 1.27) (layer B.Cu) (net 14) (status 20))
 (segment (start 42.2275 33.9725) (end 37.7825 33.9725) (width 1.27) (layer B.Cu) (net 14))
 (segment (start 37.7825 33.9725) (end 35.8775 35.8775) (width 1.27) (layer B.Cu) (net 14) (status 20))
 (segment (start 42.8625 34.6075) (end 42.2275 33.9725) (width 1.27) (layer F.Cu) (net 14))
 (segment (start 42.2275 33.9725) (end 37.7825 33.9725) (width 1.27) (layer F.Cu) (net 14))
 (segment (start 37.7825 33.9725) (end 35.8775 35.8775) (width 1.27) (layer F.Cu) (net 14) (status 20))
 (segment (start 39.0525 39.0525) (end 35.8775 35.8775) (width 2.54) (layer F.Cu) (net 14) (status 20))
 (segment (start 35.8775 43.4975) (end 40.3225 39.0525) (width 0.508) (layer B.Cu) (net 15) (status 10))
 (segment (start 40.3225 39.0525) (end 40.3225 35.8775) (width 0.508) (layer B.Cu) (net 15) (status 20))
 (segment (start 45.4025 35.8775) (end 45.4025 36.5125) (width 0.508) (layer B.Cu) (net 4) (status 30))
 (segment (start 36.5125 45.4025) (end 45.4025 36.5125) (width 0.508) (layer B.Cu) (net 4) (status 20))
 (segment (start 36.5125 46.6725) (end 36.5125 45.4025) (width 0.508) (layer B.Cu) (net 4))
 (segment (start 39.6875 49.8475) (end 36.5125 46.6725) (width 0.508) (layer B.Cu) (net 4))
 (segment (start 46.0375 49.8475) (end 39.6875 49.8475) (width 0.508) (layer B.Cu) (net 4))
 (segment (start 50.4825 54.2925) (end 46.0375 49.8475) (width 0.508) (layer B.Cu) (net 4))
 (segment (start 51.9875 54.2925) (end 50.4825 54.2925) (width 0.508) (layer B.Cu) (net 4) (status 10))
 (segment (start 52.3875 54.2925) (end 51.9875 54.2925) (width 0.508) (layer B.Cu) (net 4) (status 30))
 (segment (start 45.4025 35.8775) (end 46.6725 34.6075) (width 1.905) (layer B.Cu) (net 4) (status 10))
 (segment (start 53.0225 34.6075) (end 46.6725 34.6075) (width 1.905) (layer B.Cu) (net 4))
 (segment (start 54.2925 35.8775) (end 53.0225 34.6075) (width 1.905) (layer B.Cu) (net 4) (status 10))
 (segment (start 52.7875 54.2925) (end 52.3875 54.2925) (width 0.762) (layer F.Cu) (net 4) (status 30))
 (segment (start 46.6725 34.6075) (end 53.0225 34.6075) (width 1.905) (layer F.Cu) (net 4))
 (segment (start 53.0225 34.6075) (end 54.2925 35.8775) (width 1.905) (layer F.Cu) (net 4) (status 20))
 (segment (start 45.4025 35.8775) (end 46.6725 34.6075) (width 1.905) (layer F.Cu) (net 4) (status 10))
 (segment (start 60.0075 64.4525) (end 60.0075 61.9125) (width 0.508) (layer B.Cu) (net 2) (status 30))
 (segment (start 63.8175 51.7525) (end 65.7225 49.8475) (width 0.508) (layer B.Cu) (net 11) (status 10))
 (segment (start 65.7225 44.7675) (end 64.4525 43.4975) (width 0.508) (layer B.Cu) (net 11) (status 20))
 (segment (start 65.7225 49.8475) (end 65.7225 44.7675) (width 0.508) (layer B.Cu) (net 11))
 (segment (start 60.0075 51.7525) (end 63.8175 51.7525) (width 0.508) (layer B.Cu) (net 11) (status 30))
 (segment (start 64.4525 61.2775) (end 66.04 62.865) (width 0.508) (layer B.Cu) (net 17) (status 10))
 (segment (start 66.04 62.865) (end 66.04 69.85) (width 0.508) (layer B.Cu) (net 17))
 (segment (start 66.04 69.85) (end 65.0875 70.8025) (width 0.508) (layer B.Cu) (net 17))
 (segment (start 65.0875 70.8025) (end 62.5475 70.8025) (width 0.508) (layer B.Cu) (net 17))
 (segment (start 62.5475 70.8025) (end 58.7375 74.6125) (width 0.508) (layer B.Cu) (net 17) (status 20))
 (segment (start 35.2425 61.2775) (end 36.83 62.865) (width 0.508) (layer B.Cu) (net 17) (status 10))
 (segment (start 36.83 62.865) (end 36.83 69.85) (width 0.508) (layer B.Cu) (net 17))
 (segment (start 36.83 69.85) (end 43.4975 76.5175) (width 0.508) (layer B.Cu) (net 17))
 (segment (start 43.4975 76.5175) (end 56.8325 76.5175) (width 0.508) (layer B.Cu) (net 17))
 (segment (start 56.8325 76.5175) (end 58.7375 74.6125) (width 0.508) (layer B.Cu) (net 17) (status 20))
 (segment (start 47.625 46.99) (end 49.765 46.99) (width 0.508) (layer B.Cu) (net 1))
 (segment (start 49.765 46.99) (end 51.9875 49.2125) (width 0.508) (layer B.Cu) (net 1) (status 20))
 (segment (start 51.9875 49.2125) (end 52.3875 49.2125) (width 0.508) (layer B.Cu) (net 1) (status 30))
 (segment (start 46.99 47.625) (end 47.625 46.99) (width 0.508) (layer B.Cu) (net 1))
 (segment (start 45.085 47.625) (end 46.99 47.625) (width 0.508) (layer B.Cu) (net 1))
 (segment (start 43.4975 46.0375) (end 45.085 47.625) (width 0.508) (layer B.Cu) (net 1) (status 10))
 (segment (start 54.2925 43.4975) (end 54.2925 47.7075) (width 0.508) (layer B.Cu) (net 1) (status 10))
 (segment (start 54.2925 47.7075) (end 52.7875 49.2125) (width 0.508) (layer B.Cu) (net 1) (status 20))
 (segment (start 52.3875 49.2125) (end 52.7875 49.2125) (width 0.508) (layer B.Cu) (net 1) (status 30))
 (segment (start 54.2925 54.9275) (end 54.2925 53.2575) (width 0.508) (layer B.Cu) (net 3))
 (segment (start 54.2925 53.2575) (end 52.7875 51.7525) (width 0.508) (layer B.Cu) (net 3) (status 20))
 (segment (start 53.64151 55.57849) (end 54.2925 54.9275) (width 0.508) (layer B.Cu) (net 3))
 (segment (start 49.53 54.61) (end 50.49849 55.57849) (width 0.508) (layer B.Cu) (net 3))
 (segment (start 50.49849 55.57849) (end 53.64151 55.57849) (width 0.508) (layer B.Cu) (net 3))
 (segment (start 47.625 54.61) (end 49.53 54.61) (width 0.508) (layer B.Cu) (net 3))
 (segment (start 46.0375 56.1975) (end 47.625 54.61) (width 0.508) (layer B.Cu) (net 3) (status 10))
 (segment (start 37.7825 54.61) (end 41.91 54.61) (width 0.508) (layer B.Cu) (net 3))
 (segment (start 37.1475 55.245) (end 37.7825 54.61) (width 0.508) (layer B.Cu) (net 3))
 (segment (start 37.1475 58.1025) (end 37.1475 55.245) (width 0.508) (layer B.Cu) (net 3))
 (segment (start 38.4175 59.3725) (end 37.1475 58.1025) (width 0.508) (layer B.Cu) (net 3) (status 10))
 (segment (start 41.91 54.61) (end 43.4975 56.1975) (width 0.508) (layer B.Cu) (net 3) (status 20))
 (segment (start 43.4975 56.1975) (end 46.0375 56.1975) (width 0.508) (layer B.Cu) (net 3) (status 30))
 (segment (start 52.7875 51.7525) (end 52.3875 51.7525) (width 0.508) (layer B.Cu) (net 3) (status 30))
 (segment (start 52.3875 51.7525) (end 52.7875 51.7525) (width 0.508) (layer F.Cu) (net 3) (status 30))
 (segment (start 48.5775 48.5775) (end 43.4975 48.5775) (width 0.508) (layer B.Cu) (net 9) (status 10))
 (segment (start 50.4825 50.4825) (end 48.5775 48.5775) (width 0.508) (layer B.Cu) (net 9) (status 20))
 (segment (start 54.4895 50.4825) (end 50.4825 50.4825) (width 0.508) (layer B.Cu) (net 9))
 (segment (start 58.2995 54.2925) (end 54.4895 50.4825) (width 0.508) (layer B.Cu) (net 9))
 (segment (start 40.9575 46.0375) (end 38.4175 46.0375) (width 0.508) (layer B.Cu) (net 9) (status 30))
 (segment (start 43.4975 48.5775) (end 40.9575 46.0375) (width 0.508) (layer B.Cu) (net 9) (status 20))
 (segment (start 60.0075 54.2925) (end 58.2995 54.2925) (width 0.508) (layer B.Cu) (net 9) (status 10))
 (segment (start 60.0075 54.2925) (end 60.4075 54.2925) (width 0.508) (layer B.Cu) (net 9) (status 30)))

